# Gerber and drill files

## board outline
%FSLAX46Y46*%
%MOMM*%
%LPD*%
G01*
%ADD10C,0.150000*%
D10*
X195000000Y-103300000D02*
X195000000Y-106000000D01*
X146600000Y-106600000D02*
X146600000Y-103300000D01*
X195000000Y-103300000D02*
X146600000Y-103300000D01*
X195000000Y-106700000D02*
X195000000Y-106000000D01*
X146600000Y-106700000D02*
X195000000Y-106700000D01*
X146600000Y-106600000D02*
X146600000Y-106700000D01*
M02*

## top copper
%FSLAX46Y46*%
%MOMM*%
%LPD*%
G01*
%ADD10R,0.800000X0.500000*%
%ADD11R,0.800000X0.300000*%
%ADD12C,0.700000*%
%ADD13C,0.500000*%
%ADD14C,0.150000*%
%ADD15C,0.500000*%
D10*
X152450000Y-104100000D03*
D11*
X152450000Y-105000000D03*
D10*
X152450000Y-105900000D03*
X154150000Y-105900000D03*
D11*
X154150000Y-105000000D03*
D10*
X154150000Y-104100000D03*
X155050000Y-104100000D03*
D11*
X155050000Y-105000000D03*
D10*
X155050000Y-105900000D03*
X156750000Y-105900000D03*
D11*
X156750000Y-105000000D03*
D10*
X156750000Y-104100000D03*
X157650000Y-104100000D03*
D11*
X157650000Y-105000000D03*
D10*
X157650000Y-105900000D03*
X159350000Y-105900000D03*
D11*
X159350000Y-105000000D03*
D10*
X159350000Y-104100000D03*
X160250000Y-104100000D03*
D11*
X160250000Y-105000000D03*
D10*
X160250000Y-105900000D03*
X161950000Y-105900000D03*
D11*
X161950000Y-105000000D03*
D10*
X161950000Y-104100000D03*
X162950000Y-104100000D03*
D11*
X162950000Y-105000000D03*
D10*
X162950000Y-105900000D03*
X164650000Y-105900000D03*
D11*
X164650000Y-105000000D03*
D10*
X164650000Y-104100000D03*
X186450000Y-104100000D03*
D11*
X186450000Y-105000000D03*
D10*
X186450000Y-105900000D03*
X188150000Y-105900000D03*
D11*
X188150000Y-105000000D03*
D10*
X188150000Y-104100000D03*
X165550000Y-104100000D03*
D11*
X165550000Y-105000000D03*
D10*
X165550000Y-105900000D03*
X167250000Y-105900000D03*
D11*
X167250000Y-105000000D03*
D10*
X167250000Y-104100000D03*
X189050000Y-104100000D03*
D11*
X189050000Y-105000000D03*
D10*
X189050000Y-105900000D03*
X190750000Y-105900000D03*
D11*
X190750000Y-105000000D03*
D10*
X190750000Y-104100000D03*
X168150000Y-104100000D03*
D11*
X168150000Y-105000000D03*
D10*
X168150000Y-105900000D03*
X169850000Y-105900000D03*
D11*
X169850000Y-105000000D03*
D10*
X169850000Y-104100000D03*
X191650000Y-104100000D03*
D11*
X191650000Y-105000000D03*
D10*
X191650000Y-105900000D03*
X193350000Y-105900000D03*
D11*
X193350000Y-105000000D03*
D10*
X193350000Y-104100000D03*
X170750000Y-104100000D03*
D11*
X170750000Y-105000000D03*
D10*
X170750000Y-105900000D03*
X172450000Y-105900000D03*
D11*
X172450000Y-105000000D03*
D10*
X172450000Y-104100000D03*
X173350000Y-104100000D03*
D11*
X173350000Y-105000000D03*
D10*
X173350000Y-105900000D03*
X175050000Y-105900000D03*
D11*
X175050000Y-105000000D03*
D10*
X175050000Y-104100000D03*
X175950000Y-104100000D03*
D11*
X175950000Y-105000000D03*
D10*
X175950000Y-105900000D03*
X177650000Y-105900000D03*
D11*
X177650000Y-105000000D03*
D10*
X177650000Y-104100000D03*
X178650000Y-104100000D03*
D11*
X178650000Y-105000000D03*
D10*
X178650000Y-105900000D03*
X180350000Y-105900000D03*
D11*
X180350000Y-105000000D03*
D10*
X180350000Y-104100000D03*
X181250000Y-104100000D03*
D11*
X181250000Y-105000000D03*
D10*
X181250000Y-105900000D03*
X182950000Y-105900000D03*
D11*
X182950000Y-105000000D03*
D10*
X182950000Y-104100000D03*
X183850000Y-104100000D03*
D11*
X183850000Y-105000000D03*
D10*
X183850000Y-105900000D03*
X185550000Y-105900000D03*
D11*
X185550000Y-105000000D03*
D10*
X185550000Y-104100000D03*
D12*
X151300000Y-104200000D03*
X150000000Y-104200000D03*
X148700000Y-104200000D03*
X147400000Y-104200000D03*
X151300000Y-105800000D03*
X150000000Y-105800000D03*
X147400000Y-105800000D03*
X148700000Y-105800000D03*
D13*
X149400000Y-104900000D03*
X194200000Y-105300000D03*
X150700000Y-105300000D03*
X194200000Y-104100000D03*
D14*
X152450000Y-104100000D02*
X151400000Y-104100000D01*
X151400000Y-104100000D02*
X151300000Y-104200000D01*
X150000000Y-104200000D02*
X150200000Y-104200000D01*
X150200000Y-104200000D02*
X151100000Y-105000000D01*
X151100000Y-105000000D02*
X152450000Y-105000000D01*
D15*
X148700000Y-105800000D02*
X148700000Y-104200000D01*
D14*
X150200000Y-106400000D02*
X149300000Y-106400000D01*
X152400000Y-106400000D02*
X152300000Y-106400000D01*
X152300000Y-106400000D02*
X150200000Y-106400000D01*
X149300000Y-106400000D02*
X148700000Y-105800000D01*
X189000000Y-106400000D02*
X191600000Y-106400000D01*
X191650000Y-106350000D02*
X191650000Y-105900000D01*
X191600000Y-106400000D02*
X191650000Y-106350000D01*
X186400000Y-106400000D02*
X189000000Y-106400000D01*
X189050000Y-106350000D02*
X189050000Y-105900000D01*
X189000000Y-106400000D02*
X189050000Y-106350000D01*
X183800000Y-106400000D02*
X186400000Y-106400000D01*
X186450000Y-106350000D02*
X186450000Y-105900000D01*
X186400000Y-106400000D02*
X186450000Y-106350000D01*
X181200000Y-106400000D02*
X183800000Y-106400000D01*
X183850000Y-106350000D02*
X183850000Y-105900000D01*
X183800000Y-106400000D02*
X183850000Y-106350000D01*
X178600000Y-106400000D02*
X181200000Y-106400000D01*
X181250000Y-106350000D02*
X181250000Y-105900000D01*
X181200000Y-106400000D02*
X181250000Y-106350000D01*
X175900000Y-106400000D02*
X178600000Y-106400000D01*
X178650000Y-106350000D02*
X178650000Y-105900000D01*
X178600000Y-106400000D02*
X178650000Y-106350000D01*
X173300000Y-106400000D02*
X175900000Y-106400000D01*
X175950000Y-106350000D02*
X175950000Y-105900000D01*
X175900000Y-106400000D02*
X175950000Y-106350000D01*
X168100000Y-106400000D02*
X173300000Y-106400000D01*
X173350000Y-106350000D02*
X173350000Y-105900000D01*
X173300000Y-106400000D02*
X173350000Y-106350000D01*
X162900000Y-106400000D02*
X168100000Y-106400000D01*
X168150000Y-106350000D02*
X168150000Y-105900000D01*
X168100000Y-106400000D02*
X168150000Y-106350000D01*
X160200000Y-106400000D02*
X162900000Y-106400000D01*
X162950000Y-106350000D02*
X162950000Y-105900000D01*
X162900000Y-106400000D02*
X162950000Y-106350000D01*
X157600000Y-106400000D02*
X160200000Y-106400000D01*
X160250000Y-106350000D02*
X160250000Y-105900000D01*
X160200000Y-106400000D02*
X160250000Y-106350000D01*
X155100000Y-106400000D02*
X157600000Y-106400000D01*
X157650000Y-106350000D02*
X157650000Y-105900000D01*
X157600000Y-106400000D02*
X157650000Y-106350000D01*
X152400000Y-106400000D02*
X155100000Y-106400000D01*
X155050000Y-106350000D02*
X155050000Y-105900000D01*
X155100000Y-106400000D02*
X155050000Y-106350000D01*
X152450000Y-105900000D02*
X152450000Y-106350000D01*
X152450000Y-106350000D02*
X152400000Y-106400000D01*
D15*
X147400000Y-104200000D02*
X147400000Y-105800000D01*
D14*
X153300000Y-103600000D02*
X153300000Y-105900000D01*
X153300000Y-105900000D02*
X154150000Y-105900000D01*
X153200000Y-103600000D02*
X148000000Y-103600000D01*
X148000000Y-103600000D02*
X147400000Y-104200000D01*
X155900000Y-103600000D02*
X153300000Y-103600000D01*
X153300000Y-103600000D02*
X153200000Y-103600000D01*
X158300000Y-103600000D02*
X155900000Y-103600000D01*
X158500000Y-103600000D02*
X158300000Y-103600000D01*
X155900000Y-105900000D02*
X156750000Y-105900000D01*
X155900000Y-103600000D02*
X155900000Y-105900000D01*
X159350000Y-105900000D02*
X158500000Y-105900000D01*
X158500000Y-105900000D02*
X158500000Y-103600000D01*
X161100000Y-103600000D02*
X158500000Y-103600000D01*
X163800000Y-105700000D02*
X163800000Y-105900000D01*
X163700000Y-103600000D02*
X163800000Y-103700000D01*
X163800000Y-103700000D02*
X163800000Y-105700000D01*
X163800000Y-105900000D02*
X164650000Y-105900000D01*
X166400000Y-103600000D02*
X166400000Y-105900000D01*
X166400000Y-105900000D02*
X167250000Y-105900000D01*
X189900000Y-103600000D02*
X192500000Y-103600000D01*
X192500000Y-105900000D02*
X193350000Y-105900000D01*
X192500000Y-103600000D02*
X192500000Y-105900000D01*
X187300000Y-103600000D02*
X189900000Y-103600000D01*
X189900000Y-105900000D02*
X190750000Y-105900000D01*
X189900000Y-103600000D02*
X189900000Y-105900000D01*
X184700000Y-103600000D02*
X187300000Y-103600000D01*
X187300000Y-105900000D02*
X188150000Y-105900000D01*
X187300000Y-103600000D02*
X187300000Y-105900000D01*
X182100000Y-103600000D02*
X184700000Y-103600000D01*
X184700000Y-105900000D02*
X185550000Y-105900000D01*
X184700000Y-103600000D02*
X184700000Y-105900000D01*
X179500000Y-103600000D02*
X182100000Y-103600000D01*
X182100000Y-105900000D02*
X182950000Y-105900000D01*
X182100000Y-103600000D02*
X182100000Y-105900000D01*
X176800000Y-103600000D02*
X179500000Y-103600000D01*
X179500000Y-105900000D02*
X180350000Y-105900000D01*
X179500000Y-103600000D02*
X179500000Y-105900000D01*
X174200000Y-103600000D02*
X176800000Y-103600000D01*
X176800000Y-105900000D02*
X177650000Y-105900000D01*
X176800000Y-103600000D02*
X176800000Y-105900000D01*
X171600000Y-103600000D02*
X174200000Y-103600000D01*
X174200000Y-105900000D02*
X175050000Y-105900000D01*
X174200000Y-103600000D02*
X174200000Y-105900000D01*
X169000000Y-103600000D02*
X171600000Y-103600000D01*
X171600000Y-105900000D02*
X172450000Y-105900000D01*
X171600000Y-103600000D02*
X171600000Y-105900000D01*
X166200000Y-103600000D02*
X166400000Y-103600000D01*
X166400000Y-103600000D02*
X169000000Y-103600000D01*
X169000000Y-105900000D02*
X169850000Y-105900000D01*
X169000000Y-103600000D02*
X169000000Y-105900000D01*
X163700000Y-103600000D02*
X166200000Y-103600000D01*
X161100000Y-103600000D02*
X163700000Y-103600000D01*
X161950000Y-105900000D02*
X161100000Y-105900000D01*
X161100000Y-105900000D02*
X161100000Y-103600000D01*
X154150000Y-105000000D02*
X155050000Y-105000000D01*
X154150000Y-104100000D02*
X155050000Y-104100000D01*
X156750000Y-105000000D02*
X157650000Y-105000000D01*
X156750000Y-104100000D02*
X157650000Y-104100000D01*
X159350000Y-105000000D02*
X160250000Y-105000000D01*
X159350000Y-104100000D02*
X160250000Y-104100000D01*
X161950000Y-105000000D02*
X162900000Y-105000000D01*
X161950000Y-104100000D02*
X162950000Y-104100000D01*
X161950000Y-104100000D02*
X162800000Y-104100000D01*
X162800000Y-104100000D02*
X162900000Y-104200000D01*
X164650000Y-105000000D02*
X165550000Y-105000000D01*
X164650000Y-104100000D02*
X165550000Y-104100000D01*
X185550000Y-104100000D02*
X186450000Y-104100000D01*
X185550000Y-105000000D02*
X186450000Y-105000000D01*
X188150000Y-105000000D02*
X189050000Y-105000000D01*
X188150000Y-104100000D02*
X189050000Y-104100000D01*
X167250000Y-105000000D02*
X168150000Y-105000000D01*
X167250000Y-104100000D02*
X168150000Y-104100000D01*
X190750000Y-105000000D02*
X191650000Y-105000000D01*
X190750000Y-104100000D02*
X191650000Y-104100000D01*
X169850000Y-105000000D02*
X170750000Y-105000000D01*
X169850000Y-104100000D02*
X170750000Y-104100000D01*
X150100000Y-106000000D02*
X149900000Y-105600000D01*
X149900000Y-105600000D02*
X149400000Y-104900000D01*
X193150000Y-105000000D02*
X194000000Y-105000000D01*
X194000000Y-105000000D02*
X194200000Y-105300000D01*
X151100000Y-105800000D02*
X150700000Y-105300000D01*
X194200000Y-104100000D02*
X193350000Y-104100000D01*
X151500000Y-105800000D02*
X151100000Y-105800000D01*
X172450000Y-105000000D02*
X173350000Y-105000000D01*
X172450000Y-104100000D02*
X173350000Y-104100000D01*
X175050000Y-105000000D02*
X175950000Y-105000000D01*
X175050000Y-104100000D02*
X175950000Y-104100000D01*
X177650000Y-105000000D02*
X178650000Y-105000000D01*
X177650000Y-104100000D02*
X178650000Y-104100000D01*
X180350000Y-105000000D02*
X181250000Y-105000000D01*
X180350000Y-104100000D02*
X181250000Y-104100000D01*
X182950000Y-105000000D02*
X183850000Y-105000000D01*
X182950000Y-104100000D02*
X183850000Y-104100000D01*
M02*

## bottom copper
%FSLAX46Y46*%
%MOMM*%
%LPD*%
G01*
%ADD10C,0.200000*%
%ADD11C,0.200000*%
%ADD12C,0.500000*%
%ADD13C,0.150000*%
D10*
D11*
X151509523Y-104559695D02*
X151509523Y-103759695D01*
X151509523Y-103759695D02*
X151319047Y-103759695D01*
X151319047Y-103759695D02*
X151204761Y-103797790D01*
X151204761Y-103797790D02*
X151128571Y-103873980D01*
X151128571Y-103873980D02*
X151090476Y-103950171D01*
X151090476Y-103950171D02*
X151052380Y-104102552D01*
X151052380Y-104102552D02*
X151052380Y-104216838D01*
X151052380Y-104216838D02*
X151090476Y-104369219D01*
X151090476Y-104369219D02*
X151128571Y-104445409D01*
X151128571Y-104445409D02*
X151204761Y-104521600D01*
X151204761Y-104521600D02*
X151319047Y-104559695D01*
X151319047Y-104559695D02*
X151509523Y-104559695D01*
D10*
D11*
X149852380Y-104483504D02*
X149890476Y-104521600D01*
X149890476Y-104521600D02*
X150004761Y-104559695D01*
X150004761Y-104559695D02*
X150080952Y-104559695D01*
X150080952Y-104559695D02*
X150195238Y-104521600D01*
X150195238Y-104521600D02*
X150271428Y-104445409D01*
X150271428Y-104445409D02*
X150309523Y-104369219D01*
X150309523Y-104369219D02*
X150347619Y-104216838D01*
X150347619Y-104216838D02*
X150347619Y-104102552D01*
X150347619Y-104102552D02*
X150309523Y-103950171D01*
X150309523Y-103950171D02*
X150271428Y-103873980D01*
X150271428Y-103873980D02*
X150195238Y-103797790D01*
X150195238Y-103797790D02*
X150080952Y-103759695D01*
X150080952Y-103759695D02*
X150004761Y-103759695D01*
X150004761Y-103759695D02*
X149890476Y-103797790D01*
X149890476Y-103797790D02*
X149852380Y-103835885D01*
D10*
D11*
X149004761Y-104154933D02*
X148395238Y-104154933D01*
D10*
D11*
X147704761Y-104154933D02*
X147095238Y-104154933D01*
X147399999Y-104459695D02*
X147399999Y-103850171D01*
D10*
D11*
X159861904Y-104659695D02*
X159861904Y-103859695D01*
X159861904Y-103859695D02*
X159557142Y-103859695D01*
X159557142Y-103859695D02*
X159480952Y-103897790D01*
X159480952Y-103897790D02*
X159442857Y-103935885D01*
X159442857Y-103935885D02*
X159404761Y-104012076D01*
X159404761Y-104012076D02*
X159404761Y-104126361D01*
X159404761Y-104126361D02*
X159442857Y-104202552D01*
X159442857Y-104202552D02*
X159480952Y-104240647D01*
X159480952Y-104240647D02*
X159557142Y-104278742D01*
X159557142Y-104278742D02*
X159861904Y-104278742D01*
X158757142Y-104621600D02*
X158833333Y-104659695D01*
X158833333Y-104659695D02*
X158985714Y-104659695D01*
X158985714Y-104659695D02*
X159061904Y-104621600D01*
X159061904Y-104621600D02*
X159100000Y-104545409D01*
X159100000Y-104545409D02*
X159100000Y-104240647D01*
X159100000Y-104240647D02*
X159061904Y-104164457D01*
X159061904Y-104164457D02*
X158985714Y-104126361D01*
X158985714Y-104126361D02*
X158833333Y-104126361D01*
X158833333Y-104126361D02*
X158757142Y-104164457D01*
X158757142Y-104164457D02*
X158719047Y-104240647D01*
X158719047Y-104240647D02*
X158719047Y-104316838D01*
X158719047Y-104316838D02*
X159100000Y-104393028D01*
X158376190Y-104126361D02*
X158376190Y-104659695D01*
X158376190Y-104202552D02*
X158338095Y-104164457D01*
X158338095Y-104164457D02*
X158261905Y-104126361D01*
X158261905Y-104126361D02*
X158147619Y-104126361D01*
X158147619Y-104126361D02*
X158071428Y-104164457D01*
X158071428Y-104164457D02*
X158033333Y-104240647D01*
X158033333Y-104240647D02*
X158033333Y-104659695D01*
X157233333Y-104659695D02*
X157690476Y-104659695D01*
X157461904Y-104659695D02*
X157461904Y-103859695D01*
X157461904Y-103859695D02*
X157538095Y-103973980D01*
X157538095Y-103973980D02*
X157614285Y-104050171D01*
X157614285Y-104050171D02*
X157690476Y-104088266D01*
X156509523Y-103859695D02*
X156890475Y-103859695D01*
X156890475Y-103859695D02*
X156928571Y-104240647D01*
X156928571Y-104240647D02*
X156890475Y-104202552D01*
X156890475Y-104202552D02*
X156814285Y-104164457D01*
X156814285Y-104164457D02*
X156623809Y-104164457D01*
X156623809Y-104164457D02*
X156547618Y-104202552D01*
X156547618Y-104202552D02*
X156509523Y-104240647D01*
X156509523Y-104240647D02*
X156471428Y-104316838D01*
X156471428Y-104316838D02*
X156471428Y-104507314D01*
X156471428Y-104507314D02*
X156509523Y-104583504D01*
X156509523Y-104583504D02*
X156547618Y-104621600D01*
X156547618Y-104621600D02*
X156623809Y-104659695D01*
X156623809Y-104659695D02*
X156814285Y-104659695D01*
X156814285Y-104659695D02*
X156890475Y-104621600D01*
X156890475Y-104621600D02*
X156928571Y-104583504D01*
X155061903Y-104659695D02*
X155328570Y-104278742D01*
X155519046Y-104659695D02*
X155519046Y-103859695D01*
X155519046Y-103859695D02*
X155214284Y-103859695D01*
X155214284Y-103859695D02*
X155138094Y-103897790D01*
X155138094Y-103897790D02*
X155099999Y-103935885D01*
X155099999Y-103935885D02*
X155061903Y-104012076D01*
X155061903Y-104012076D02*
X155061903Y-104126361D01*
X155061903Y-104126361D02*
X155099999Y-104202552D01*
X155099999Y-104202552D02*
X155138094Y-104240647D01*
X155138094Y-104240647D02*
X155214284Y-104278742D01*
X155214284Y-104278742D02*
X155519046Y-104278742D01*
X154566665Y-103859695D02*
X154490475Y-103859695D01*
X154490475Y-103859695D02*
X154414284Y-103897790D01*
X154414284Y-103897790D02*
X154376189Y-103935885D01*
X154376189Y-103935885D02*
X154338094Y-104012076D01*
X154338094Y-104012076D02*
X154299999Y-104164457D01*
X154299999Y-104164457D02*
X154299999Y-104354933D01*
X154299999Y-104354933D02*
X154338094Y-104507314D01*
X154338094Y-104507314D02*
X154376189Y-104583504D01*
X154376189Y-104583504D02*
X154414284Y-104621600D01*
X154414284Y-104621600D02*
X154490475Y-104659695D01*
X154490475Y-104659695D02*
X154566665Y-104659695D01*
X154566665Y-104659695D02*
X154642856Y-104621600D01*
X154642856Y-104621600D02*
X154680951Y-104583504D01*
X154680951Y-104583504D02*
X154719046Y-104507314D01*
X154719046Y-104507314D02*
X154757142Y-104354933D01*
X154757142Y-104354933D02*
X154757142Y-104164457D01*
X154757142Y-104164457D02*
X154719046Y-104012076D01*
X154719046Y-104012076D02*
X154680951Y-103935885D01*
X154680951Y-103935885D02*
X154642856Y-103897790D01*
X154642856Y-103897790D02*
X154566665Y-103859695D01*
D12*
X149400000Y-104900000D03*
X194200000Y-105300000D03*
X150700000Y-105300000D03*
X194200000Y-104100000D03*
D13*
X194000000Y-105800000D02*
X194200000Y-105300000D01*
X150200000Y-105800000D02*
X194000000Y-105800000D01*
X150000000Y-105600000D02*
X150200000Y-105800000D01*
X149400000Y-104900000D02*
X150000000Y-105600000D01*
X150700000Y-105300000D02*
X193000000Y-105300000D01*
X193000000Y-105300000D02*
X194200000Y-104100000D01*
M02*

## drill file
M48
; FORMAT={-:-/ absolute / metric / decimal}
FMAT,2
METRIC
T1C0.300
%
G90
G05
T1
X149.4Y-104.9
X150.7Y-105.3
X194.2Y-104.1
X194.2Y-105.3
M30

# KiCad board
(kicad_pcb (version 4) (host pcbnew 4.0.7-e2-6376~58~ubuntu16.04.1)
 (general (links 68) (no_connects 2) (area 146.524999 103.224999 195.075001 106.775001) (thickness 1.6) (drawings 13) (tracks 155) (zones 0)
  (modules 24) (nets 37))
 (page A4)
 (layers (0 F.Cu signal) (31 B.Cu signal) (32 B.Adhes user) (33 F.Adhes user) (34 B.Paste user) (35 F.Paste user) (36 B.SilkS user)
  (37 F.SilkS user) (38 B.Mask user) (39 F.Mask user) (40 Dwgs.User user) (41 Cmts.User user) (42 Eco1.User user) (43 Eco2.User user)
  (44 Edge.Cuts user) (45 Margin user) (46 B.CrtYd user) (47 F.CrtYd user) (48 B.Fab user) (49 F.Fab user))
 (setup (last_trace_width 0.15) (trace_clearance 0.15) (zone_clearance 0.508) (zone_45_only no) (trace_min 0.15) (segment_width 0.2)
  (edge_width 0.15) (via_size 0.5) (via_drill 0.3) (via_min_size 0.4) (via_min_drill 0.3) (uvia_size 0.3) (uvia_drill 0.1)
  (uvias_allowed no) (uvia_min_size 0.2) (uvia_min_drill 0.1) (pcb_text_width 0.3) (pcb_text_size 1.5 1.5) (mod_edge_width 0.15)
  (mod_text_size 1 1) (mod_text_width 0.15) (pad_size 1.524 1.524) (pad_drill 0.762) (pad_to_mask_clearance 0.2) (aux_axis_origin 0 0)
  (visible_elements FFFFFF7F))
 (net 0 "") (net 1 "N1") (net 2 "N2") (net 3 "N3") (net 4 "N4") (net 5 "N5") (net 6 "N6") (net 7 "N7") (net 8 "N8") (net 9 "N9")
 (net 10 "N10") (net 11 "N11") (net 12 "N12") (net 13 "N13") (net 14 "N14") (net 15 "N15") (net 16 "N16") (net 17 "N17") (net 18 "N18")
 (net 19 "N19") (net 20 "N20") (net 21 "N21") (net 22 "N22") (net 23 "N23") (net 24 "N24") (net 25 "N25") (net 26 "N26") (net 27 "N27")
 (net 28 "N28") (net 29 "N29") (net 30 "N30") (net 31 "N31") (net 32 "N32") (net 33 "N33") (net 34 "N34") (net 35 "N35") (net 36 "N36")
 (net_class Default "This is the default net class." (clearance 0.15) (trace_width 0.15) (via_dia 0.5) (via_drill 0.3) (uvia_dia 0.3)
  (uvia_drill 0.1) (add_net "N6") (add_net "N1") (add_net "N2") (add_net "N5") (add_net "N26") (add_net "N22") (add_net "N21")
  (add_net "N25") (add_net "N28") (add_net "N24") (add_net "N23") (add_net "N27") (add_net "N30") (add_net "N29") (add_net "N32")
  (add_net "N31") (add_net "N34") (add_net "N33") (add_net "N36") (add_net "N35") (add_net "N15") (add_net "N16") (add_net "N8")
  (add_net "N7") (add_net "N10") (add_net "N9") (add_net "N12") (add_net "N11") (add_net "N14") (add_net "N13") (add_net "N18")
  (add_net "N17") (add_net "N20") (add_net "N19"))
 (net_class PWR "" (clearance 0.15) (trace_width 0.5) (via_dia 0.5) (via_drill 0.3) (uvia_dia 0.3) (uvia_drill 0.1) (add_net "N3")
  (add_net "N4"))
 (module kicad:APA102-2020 (layer F.Cu) (at 153.3 105)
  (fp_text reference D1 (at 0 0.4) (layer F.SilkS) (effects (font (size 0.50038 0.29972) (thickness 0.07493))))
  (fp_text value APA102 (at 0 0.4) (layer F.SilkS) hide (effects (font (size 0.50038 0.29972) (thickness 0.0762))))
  (pad 2 smd rect (at -0.85 -0.9) (size 0.8 0.5) (layers F.Cu F.Paste F.Mask) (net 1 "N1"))
  (pad 3 smd rect (at -0.85 0) (size 0.8 0.3) (layers F.Cu F.Paste F.Mask) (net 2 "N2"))
  (pad 4 smd rect (at -0.85 0.9) (size 0.8 0.5) (layers F.Cu F.Paste F.Mask) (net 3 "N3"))
  (pad 5 smd rect (at 0.85 0.9) (size 0.8 0.5) (layers F.Cu F.Paste F.Mask) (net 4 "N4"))
  (pad 6 smd rect (at 0.85 0) (size 0.8 0.3) (layers F.Cu F.Paste F.Mask) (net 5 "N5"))
  (pad 1 smd rect (at 0.85 -0.9) (size 0.8 0.5) (layers F.Cu F.Paste F.Mask) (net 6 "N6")))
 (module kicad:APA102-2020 (layer F.Cu) (at 155.9 105)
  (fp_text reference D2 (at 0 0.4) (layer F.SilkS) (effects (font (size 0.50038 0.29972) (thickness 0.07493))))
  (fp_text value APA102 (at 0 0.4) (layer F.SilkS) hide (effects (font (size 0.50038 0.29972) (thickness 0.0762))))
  (pad 2 smd rect (at -0.85 -0.9) (size 0.8 0.5) (layers F.Cu F.Paste F.Mask) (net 6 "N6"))
  (pad 3 smd rect (at -0.85 0) (size 0.8 0.3) (layers F.Cu F.Paste F.Mask) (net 5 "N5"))
  (pad 4 smd rect (at -0.85 0.9) (size 0.8 0.5) (layers F.Cu F.Paste F.Mask) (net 3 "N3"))
  (pad 5 smd rect (at 0.85 0.9) (size 0.8 0.5) (layers F.Cu F.Paste F.Mask) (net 4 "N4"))
  (pad 6 smd rect (at 0.85 0) (size 0.8 0.3) (layers F.Cu F.Paste F.Mask) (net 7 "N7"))
  (pad 1 smd rect (at 0.85 -0.9) (size 0.8 0.5) (layers F.Cu F.Paste F.Mask) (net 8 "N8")))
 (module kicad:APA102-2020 (layer F.Cu) (at 158.5 105)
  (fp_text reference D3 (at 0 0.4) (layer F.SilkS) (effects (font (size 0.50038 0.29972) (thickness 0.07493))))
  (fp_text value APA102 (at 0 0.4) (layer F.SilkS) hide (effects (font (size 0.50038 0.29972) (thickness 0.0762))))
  (pad 2 smd rect (at -0.85 -0.9) (size 0.8 0.5) (layers F.Cu F.Paste F.Mask) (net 8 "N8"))
  (pad 3 smd rect (at -0.85 0) (size 0.8 0.3) (layers F.Cu F.Paste F.Mask) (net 7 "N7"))
  (pad 4 smd rect (at -0.85 0.9) (size 0.8 0.5) (layers F.Cu F.Paste F.Mask) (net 3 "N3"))
  (pad 5 smd rect (at 0.85 0.9) (size 0.8 0.5) (layers F.Cu F.Paste F.Mask) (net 4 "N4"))
  (pad 6 smd rect (at 0.85 0) (size 0.8 0.3) (layers F.Cu F.Paste F.Mask) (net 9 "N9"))
  (pad 1 smd rect (at 0.85 -0.9) (size 0.8 0.5) (layers F.Cu F.Paste F.Mask) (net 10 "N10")))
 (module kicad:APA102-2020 (layer F.Cu) (at 161.1 105)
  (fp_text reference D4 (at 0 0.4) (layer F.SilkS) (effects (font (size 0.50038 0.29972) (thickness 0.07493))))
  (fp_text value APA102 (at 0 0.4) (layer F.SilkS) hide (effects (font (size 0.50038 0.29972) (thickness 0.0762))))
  (pad 2 smd rect (at -0.85 -0.9) (size 0.8 0.5) (layers F.Cu F.Paste F.Mask) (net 10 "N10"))
  (pad 3 smd rect (at -0.85 0) (size 0.8 0.3) (layers F.Cu F.Paste F.Mask) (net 9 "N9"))
  (pad 4 smd rect (at -0.85 0.9) (size 0.8 0.5) (layers F.Cu F.Paste F.Mask) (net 3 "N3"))
  (pad 5 smd rect (at 0.85 0.9) (size 0.8 0.5) (layers F.Cu F.Paste F.Mask) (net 4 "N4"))
  (pad 6 smd rect (at 0.85 0) (size 0.8 0.3) (layers F.Cu F.Paste F.Mask) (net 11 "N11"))
  (pad 1 smd rect (at 0.85 -0.9) (size 0.8 0.5) (layers F.Cu F.Paste F.Mask) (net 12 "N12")))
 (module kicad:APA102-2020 (layer F.Cu) (at 163.8 105)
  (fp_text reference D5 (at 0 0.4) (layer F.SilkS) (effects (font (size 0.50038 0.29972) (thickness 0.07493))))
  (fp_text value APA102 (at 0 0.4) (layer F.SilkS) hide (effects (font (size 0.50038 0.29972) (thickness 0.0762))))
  (pad 2 smd rect (at -0.85 -0.9) (size 0.8 0.5) (layers F.Cu F.Paste F.Mask) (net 12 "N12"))
  (pad 3 smd rect (at -0.85 0) (size 0.8 0.3) (layers F.Cu F.Paste F.Mask) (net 11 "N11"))
  (pad 4 smd rect (at -0.85 0.9) (size 0.8 0.5) (layers F.Cu F.Paste F.Mask) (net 3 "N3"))
  (pad 5 smd rect (at 0.85 0.9) (size 0.8 0.5) (layers F.Cu F.Paste F.Mask) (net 4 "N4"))
  (pad 6 smd rect (at 0.85 0) (size 0.8 0.3) (layers F.Cu F.Paste F.Mask) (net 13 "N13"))
  (pad 1 smd rect (at 0.85 -0.9) (size 0.8 0.5) (layers F.Cu F.Paste F.Mask) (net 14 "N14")))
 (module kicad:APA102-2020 (layer F.Cu) (at 187.3 105)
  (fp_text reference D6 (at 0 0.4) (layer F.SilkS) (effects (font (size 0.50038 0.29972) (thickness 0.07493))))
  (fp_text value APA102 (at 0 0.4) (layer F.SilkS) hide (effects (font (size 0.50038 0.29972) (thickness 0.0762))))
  (pad 2 smd rect (at -0.85 -0.9) (size 0.8 0.5) (layers F.Cu F.Paste F.Mask) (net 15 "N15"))
  (pad 3 smd rect (at -0.85 0) (size 0.8 0.3) (layers F.Cu F.Paste F.Mask) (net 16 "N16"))
  (pad 4 smd rect (at -0.85 0.9) (size 0.8 0.5) (layers F.Cu F.Paste F.Mask) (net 3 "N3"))
  (pad 5 smd rect (at 0.85 0.9) (size 0.8 0.5) (layers F.Cu F.Paste F.Mask) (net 4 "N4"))
  (pad 6 smd rect (at 0.85 0) (size 0.8 0.3) (layers F.Cu F.Paste F.Mask) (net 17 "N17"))
  (pad 1 smd rect (at 0.85 -0.9) (size 0.8 0.5) (layers F.Cu F.Paste F.Mask) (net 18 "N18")))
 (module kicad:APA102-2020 (layer F.Cu) (at 166.4 105)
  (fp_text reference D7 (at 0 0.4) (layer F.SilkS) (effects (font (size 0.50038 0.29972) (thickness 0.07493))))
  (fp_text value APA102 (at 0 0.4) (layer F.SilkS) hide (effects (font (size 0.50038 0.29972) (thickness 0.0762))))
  (pad 2 smd rect (at -0.85 -0.9) (size 0.8 0.5) (layers F.Cu F.Paste F.Mask) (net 14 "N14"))
  (pad 3 smd rect (at -0.85 0) (size 0.8 0.3) (layers F.Cu F.Paste F.Mask) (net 13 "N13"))
  (pad 4 smd rect (at -0.85 0.9) (size 0.8 0.5) (layers F.Cu F.Paste F.Mask) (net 3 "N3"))
  (pad 5 smd rect (at 0.85 0.9) (size 0.8 0.5) (layers F.Cu F.Paste F.Mask) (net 4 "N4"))
  (pad 6 smd rect (at 0.85 0) (size 0.8 0.3) (layers F.Cu F.Paste F.Mask) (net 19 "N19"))
  (pad 1 smd rect (at 0.85 -0.9) (size 0.8 0.5) (layers F.Cu F.Paste F.Mask) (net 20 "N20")))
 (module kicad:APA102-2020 (layer F.Cu) (at 189.9 105)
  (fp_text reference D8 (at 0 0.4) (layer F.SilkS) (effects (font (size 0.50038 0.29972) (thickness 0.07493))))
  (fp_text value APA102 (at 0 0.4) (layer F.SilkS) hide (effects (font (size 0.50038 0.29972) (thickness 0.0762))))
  (pad 2 smd rect (at -0.85 -0.9) (size 0.8 0.5) (layers F.Cu F.Paste F.Mask) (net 18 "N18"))
  (pad 3 smd rect (at -0.85 0) (size 0.8 0.3) (layers F.Cu F.Paste F.Mask) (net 17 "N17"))
  (pad 4 smd rect (at -0.85 0.9) (size 0.8 0.5) (layers F.Cu F.Paste F.Mask) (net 3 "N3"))
  (pad 5 smd rect (at 0.85 0.9) (size 0.8 0.5) (layers F.Cu F.Paste F.Mask) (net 4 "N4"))
  (pad 6 smd rect (at 0.85 0) (size 0.8 0.3) (layers F.Cu F.Paste F.Mask) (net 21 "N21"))
  (pad 1 smd rect (at 0.85 -0.9) (size 0.8 0.5) (layers F.Cu F.Paste F.Mask) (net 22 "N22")))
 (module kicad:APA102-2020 (layer F.Cu) (at 169 105)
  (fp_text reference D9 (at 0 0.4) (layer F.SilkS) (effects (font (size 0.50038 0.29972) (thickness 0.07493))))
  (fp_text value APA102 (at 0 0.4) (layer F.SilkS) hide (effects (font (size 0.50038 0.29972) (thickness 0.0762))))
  (pad 2 smd rect (at -0.85 -0.9) (size 0.8 0.5) (layers F.Cu F.Paste F.Mask) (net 20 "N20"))
  (pad 3 smd rect (at -0.85 0) (size 0.8 0.3) (layers F.Cu F.Paste F.Mask) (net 19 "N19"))
  (pad 4 smd rect (at -0.85 0.9) (size 0.8 0.5) (layers F.Cu F.Paste F.Mask) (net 3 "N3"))
  (pad 5 smd rect (at 0.85 0.9) (size 0.8 0.5) (layers F.Cu F.Paste F.Mask) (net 4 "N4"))
  (pad 6 smd rect (at 0.85 0) (size 0.8 0.3) (layers F.Cu F.Paste F.Mask) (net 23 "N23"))
  (pad 1 smd rect (at 0.85 -0.9) (size 0.8 0.5) (layers F.Cu F.Paste F.Mask) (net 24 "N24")))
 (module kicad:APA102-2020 (layer F.Cu) (at 192.5 105)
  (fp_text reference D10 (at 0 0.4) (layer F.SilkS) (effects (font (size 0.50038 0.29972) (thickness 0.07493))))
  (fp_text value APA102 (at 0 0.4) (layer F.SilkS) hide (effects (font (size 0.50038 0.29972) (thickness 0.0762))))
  (pad 2 smd rect (at -0.85 -0.9) (size 0.8 0.5) (layers F.Cu F.Paste F.Mask) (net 22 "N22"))
  (pad 3 smd rect (at -0.85 0) (size 0.8 0.3) (layers F.Cu F.Paste F.Mask) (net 21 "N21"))
  (pad 4 smd rect (at -0.85 0.9) (size 0.8 0.5) (layers F.Cu F.Paste F.Mask) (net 3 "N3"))
  (pad 5 smd rect (at 0.85 0.9) (size 0.8 0.5) (layers F.Cu F.Paste F.Mask) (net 4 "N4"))
  (pad 6 smd rect (at 0.85 0) (size 0.8 0.3) (layers F.Cu F.Paste F.Mask) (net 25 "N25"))
  (pad 1 smd rect (at 0.85 -0.9) (size 0.8 0.5) (layers F.Cu F.Paste F.Mask) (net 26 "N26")))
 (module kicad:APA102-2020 (layer F.Cu) (at 171.6 105)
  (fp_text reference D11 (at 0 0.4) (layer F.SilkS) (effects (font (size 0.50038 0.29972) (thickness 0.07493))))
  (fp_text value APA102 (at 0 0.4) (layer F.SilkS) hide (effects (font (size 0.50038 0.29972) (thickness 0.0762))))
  (pad 2 smd rect (at -0.85 -0.9) (size 0.8 0.5) (layers F.Cu F.Paste F.Mask) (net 24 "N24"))
  (pad 3 smd rect (at -0.85 0) (size 0.8 0.3) (layers F.Cu F.Paste F.Mask) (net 23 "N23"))
  (pad 4 smd rect (at -0.85 0.9) (size 0.8 0.5) (layers F.Cu F.Paste F.Mask) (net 3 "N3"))
  (pad 5 smd rect (at 0.85 0.9) (size 0.8 0.5) (layers F.Cu F.Paste F.Mask) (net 4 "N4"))
  (pad 6 smd rect (at 0.85 0) (size 0.8 0.3) (layers F.Cu F.Paste F.Mask) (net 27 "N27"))
  (pad 1 smd rect (at 0.85 -0.9) (size 0.8 0.5) (layers F.Cu F.Paste F.Mask) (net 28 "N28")))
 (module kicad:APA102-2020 (layer F.Cu) (at 174.2 105)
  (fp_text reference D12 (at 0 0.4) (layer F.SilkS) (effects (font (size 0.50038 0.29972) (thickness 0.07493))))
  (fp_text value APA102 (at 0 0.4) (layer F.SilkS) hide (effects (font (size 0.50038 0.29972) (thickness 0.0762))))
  (pad 2 smd rect (at -0.85 -0.9) (size 0.8 0.5) (layers F.Cu F.Paste F.Mask) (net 28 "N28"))
  (pad 3 smd rect (at -0.85 0) (size 0.8 0.3) (layers F.Cu F.Paste F.Mask) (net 27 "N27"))
  (pad 4 smd rect (at -0.85 0.9) (size 0.8 0.5) (layers F.Cu F.Paste F.Mask) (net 3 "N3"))
  (pad 5 smd rect (at 0.85 0.9) (size 0.8 0.5) (layers F.Cu F.Paste F.Mask) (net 4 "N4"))
  (pad 6 smd rect (at 0.85 0) (size 0.8 0.3) (layers F.Cu F.Paste F.Mask) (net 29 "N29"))
  (pad 1 smd rect (at 0.85 -0.9) (size 0.8 0.5) (layers F.Cu F.Paste F.Mask) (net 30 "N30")))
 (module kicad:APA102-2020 (layer F.Cu) (at 176.8 105)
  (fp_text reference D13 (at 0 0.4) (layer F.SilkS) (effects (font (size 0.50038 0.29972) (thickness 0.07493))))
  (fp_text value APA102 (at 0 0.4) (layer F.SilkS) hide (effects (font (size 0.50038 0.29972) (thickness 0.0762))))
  (pad 2 smd rect (at -0.85 -0.9) (size 0.8 0.5) (layers F.Cu F.Paste F.Mask) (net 30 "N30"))
  (pad 3 smd rect (at -0.85 0) (size 0.8 0.3) (layers F.Cu F.Paste F.Mask) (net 29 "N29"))
  (pad 4 smd rect (at -0.85 0.9) (size 0.8 0.5) (layers F.Cu F.Paste F.Mask) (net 3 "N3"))
  (pad 5 smd rect (at 0.85 0.9) (size 0.8 0.5) (layers F.Cu F.Paste F.Mask) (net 4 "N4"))
  (pad 6 smd rect (at 0.85 0) (size 0.8 0.3) (layers F.Cu F.Paste F.Mask) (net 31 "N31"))
  (pad 1 smd rect (at 0.85 -0.9) (size 0.8 0.5) (layers F.Cu F.Paste F.Mask) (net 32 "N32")))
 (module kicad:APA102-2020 (layer F.Cu) (at 179.5 105)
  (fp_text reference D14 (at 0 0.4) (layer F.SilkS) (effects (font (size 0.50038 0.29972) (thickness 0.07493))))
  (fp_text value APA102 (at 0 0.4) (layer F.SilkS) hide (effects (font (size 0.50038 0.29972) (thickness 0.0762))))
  (pad 2 smd rect (at -0.85 -0.9) (size 0.8 0.5) (layers F.Cu F.Paste F.Mask) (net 32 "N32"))
  (pad 3 smd rect (at -0.85 0) (size 0.8 0.3) (layers F.Cu F.Paste F.Mask) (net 31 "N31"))
  (pad 4 smd rect (at -0.85 0.9) (size 0.8 0.5) (layers F.Cu F.Paste F.Mask) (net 3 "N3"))
  (pad 5 smd rect (at 0.85 0.9) (size 0.8 0.5) (layers F.Cu F.Paste F.Mask) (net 4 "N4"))
  (pad 6 smd rect (at 0.85 0) (size 0.8 0.3) (layers F.Cu F.Paste F.Mask) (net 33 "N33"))
  (pad 1 smd rect (at 0.85 -0.9) (size 0.8 0.5) (layers F.Cu F.Paste F.Mask) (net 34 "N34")))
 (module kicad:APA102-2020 (layer F.Cu) (at 182.1 105)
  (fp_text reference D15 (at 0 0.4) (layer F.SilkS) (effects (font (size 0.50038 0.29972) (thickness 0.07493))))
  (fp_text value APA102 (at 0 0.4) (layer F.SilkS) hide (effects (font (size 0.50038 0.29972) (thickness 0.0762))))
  (pad 2 smd rect (at -0.85 -0.9) (size 0.8 0.5) (layers F.Cu F.Paste F.Mask) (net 34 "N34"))
  (pad 3 smd rect (at -0.85 0) (size 0.8 0.3) (layers F.Cu F.Paste F.Mask) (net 33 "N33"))
  (pad 4 smd rect (at -0.85 0.9) (size 0.8 0.5) (layers F.Cu F.Paste F.Mask) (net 3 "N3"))
  (pad 5 smd rect (at 0.85 0.9) (size 0.8 0.5) (layers F.Cu F.Paste F.Mask) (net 4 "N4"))
  (pad 6 smd rect (at 0.85 0) (size 0.8 0.3) (layers F.Cu F.Paste F.Mask) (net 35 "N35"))
  (pad 1 smd rect (at 0.85 -0.9) (size 0.8 0.5) (layers F.Cu F.Paste F.Mask) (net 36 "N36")))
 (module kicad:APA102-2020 (layer F.Cu) (at 184.7 105)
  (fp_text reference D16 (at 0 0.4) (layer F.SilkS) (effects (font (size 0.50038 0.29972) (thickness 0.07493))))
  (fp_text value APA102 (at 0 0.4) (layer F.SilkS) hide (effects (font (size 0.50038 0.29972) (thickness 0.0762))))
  (pad 2 smd rect (at -0.85 -0.9) (size 0.8 0.5) (layers F.Cu F.Paste F.Mask) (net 36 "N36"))
  (pad 3 smd rect (at -0.85 0) (size 0.8 0.3) (layers F.Cu F.Paste F.Mask) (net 35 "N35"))
  (pad 4 smd rect (at -0.85 0.9) (size 0.8 0.5) (layers F.Cu F.Paste F.Mask) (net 3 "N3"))
  (pad 5 smd rect (at 0.85 0.9) (size 0.8 0.5) (layers F.Cu F.Paste F.Mask) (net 4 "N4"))
  (pad 6 smd rect (at 0.85 0) (size 0.8 0.3) (layers F.Cu F.Paste F.Mask) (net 16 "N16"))
  (pad 1 smd rect (at 0.85 -0.9) (size 0.8 0.5) (layers F.Cu F.Paste F.Mask) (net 15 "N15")))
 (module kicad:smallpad (layer F.Cu) (at 151.3 104.2)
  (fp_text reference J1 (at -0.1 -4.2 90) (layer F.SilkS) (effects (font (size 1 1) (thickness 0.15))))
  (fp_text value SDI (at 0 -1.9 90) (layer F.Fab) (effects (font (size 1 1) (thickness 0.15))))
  (pad 1 smd circle (at 0 0) (size 0.7 0.7) (layers F.Cu F.Paste F.Mask) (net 1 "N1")))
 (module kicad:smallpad (layer F.Cu) (at 150 104.2)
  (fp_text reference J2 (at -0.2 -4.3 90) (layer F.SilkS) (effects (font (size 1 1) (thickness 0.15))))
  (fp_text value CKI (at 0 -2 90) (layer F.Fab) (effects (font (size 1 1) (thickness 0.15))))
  (pad 1 smd circle (at 0 0) (size 0.7 0.7) (layers F.Cu F.Paste F.Mask) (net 2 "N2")))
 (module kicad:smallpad (layer F.Cu) (at 148.7 104.2)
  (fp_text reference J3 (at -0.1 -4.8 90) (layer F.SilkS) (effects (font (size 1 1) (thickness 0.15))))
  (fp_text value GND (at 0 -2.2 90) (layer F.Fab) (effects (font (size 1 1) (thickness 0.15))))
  (pad 1 smd circle (at 0 0) (size 0.7 0.7) (layers F.Cu F.Paste F.Mask) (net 3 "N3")))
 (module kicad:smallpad (layer F.Cu) (at 147.4 104.2)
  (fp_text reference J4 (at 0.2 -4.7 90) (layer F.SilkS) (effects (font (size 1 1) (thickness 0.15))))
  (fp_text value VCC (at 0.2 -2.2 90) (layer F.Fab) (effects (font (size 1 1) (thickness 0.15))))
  (pad 1 smd circle (at 0 0) (size 0.7 0.7) (layers F.Cu F.Paste F.Mask) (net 4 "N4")))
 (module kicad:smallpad (layer F.Cu) (at 151.3 105.8)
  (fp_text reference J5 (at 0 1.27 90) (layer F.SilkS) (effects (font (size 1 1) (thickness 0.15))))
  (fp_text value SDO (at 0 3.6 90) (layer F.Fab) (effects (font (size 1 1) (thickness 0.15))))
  (pad 1 smd circle (at 0 0) (size 0.7 0.7) (layers F.Cu F.Paste F.Mask) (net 26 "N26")))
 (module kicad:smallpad (layer F.Cu) (at 150 105.8)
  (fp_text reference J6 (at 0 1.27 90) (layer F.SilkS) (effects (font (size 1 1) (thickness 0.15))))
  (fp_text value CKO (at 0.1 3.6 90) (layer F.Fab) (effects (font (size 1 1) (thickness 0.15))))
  (pad 1 smd circle (at 0 0) (size 0.7 0.7) (layers F.Cu F.Paste F.Mask) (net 25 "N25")))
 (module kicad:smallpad (layer F.Cu) (at 147.4 105.8)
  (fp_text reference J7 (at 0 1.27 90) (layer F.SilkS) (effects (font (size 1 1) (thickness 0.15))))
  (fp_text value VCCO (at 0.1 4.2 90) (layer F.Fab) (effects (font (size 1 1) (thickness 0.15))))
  (pad 1 smd circle (at 0 0) (size 0.7 0.7) (layers F.Cu F.Paste F.Mask) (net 4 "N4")))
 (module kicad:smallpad (layer F.Cu) (at 148.7 105.8)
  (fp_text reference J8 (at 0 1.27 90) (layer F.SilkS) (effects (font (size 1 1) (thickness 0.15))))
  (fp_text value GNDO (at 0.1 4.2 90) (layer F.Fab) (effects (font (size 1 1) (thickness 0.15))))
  (pad 1 smd circle (at 0 0) (size 0.7 0.7) (layers F.Cu F.Paste F.Mask) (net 3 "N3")))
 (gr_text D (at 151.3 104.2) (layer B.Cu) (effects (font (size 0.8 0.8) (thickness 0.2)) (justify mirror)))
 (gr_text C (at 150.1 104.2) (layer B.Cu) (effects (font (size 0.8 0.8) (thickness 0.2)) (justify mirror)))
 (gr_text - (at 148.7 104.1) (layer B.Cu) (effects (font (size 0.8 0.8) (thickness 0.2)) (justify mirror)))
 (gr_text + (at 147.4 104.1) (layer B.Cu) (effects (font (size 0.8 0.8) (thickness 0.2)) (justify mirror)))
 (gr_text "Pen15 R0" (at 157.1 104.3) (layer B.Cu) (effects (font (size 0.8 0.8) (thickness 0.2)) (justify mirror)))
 (gr_line (start 195 103.3) (end 195 106) (angle 90) (layer Edge.Cuts) (width 0.15))
 (gr_line (start 146.6 106.6) (end 146.6 103.3) (angle 90) (layer Edge.Cuts) (width 0.15))
 (gr_line (start 195 103.3) (end 146.6 103.3) (angle 90) (layer Edge.Cuts) (width 0.15))
 (gr_line (start 195 106.7) (end 195 106) (angle 90) (layer Edge.Cuts) (width 0.15))
 (gr_line (start 146.6 106.7) (end 195 106.7) (angle 90) (layer Edge.Cuts) (width 0.15))
 (gr_line (start 146.6 106.6) (end 146.6 106.7) (angle 90) (layer Edge.Cuts) (width 0.15))
 (segment (start 152.45 104.1) (end 151.4 104.1) (width 0.15) (layer F.Cu) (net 1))
 (segment (start 151.4 104.1) (end 151.3 104.2) (width 0.15) (layer F.Cu) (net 1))
 (segment (start 150 104.2) (end 150.2 104.2) (width 0.15) (layer F.Cu) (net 2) (status 30))
 (segment (start 150.2 104.2) (end 151.1 105) (width 0.15) (layer F.Cu) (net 2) (status 10))
 (segment (start 151.1 105) (end 152.45 105) (width 0.15) (layer F.Cu) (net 2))
 (segment (start 148.7 105.8) (end 148.7 104.2) (width 0.5) (layer F.Cu) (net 3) (status 10))
 (segment (start 150.2 106.4) (end 149.3 106.4) (width 0.15) (layer F.Cu) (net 3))
 (segment (start 152.4 106.4) (end 152.3 106.4) (width 0.15) (layer F.Cu) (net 3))
 (segment (start 152.3 106.4) (end 150.2 106.4) (width 0.15) (layer F.Cu) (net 3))
 (segment (start 149.3 106.4) (end 148.7 105.8) (width 0.15) (layer F.Cu) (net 3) (status 20))
 (segment (start 189 106.4) (end 191.6 106.4) (width 0.15) (layer F.Cu) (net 3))
 (segment (start 191.65 106.35) (end 191.65 105.9) (width 0.15) (layer F.Cu) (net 3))
 (segment (start 191.6 106.4) (end 191.65 106.35) (width 0.15) (layer F.Cu) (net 3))
 (segment (start 186.4 106.4) (end 189 106.4) (width 0.15) (layer F.Cu) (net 3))
 (segment (start 189.05 106.35) (end 189.05 105.9) (width 0.15) (layer F.Cu) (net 3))
 (segment (start 189 106.4) (end 189.05 106.35) (width 0.15) (layer F.Cu) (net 3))
 (segment (start 183.8 106.4) (end 186.4 106.4) (width 0.15) (layer F.Cu) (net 3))
 (segment (start 186.45 106.35) (end 186.45 105.9) (width 0.15) (layer F.Cu) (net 3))
 (segment (start 186.4 106.4) (end 186.45 106.35) (width 0.15) (layer F.Cu) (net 3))
 (segment (start 181.2 106.4) (end 183.8 106.4) (width 0.15) (layer F.Cu) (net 3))
 (segment (start 183.85 106.35) (end 183.85 105.9) (width 0.15) (layer F.Cu) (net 3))
 (segment (start 183.8 106.4) (end 183.85 106.35) (width 0.15) (layer F.Cu) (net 3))
 (segment (start 178.6 106.4) (end 181.2 106.4) (width 0.15) (layer F.Cu) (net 3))
 (segment (start 181.25 106.35) (end 181.25 105.9) (width 0.15) (layer F.Cu) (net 3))
 (segment (start 181.2 106.4) (end 181.25 106.35) (width 0.15) (layer F.Cu) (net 3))
 (segment (start 175.9 106.4) (end 178.6 106.4) (width 0.15) (layer F.Cu) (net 3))
 (segment (start 178.65 106.35) (end 178.65 105.9) (width 0.15) (layer F.Cu) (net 3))
 (segment (start 178.6 106.4) (end 178.65 106.35) (width 0.15) (layer F.Cu) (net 3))
 (segment (start 173.3 106.4) (end 175.9 106.4) (width 0.15) (layer F.Cu) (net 3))
 (segment (start 175.95 106.35) (end 175.95 105.9) (width 0.15) (layer F.Cu) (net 3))
 (segment (start 175.9 106.4) (end 175.95 106.35) (width 0.15) (layer F.Cu) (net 3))
 (segment (start 168.1 106.4) (end 173.3 106.4) (width 0.15) (layer F.Cu) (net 3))
 (segment (start 173.35 106.35) (end 173.35 105.9) (width 0.15) (layer F.Cu) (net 3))
 (segment (start 173.3 106.4) (end 173.35 106.35) (width 0.15) (layer F.Cu) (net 3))
 (segment (start 162.9 106.4) (end 168.1 106.4) (width 0.15) (layer F.Cu) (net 3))
 (segment (start 168.15 106.35) (end 168.15 105.9) (width 0.15) (layer F.Cu) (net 3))
 (segment (start 168.1 106.4) (end 168.15 106.35) (width 0.15) (layer F.Cu) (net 3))
 (segment (start 160.2 106.4) (end 162.9 106.4) (width 0.15) (layer F.Cu) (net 3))
 (segment (start 162.95 106.35) (end 162.95 105.9) (width 0.15) (layer F.Cu) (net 3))
 (segment (start 162.9 106.4) (end 162.95 106.35) (width 0.15) (layer F.Cu) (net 3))
 (segment (start 157.6 106.4) (end 160.2 106.4) (width 0.15) (layer F.Cu) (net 3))
 (segment (start 160.25 106.35) (end 160.25 105.9) (width 0.15) (layer F.Cu) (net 3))
 (segment (start 160.2 106.4) (end 160.25 106.35) (width 0.15) (layer F.Cu) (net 3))
 (segment (start 155.1 106.4) (end 157.6 106.4) (width 0.15) (layer F.Cu) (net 3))
 (segment (start 157.65 106.35) (end 157.65 105.9) (width 0.15) (layer F.Cu) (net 3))
 (segment (start 157.6 106.4) (end 157.65 106.35) (width 0.15) (layer F.Cu) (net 3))
 (segment (start 152.4 106.4) (end 155.1 106.4) (width 0.15) (layer F.Cu) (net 3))
 (segment (start 155.05 106.35) (end 155.05 105.9) (width 0.15) (layer F.Cu) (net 3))
 (segment (start 155.1 106.4) (end 155.05 106.35) (width 0.15) (layer F.Cu) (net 3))
 (segment (start 152.45 105.9) (end 152.45 106.35) (width 0.15) (layer F.Cu) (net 3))
 (segment (start 152.45 106.35) (end 152.4 106.4) (width 0.15) (layer F.Cu) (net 3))
 (segment (start 147.4 104.2) (end 147.4 105.8) (width 0.5) (layer F.Cu) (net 4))
 (segment (start 153.3 103.6) (end 153.3 105.9) (width 0.15) (layer F.Cu) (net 4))
 (segment (start 153.3 105.9) (end 154.15 105.9) (width 0.15) (layer F.Cu) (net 4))
 (segment (start 153.2 103.6) (end 148 103.6) (width 0.15) (layer F.Cu) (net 4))
 (segment (start 148 103.6) (end 147.4 104.2) (width 0.15) (layer F.Cu) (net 4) (status 20))
 (segment (start 155.9 103.6) (end 153.3 103.6) (width 0.15) (layer F.Cu) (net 4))
 (segment (start 153.3 103.6) (end 153.2 103.6) (width 0.15) (layer F.Cu) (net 4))
 (segment (start 158.3 103.6) (end 155.9 103.6) (width 0.15) (layer F.Cu) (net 4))
 (segment (start 158.5 103.6) (end 158.3 103.6) (width 0.15) (layer F.Cu) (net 4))
 (segment (start 155.9 105.9) (end 156.75 105.9) (width 0.15) (layer F.Cu) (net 4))
 (segment (start 155.9 103.6) (end 155.9 105.9) (width 0.15) (layer F.Cu) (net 4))
 (segment (start 159.35 105.9) (end 158.5 105.9) (width 0.15) (layer F.Cu) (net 4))
 (segment (start 158.5 105.9) (end 158.5 103.6) (width 0.15) (layer F.Cu) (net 4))
 (segment (start 161.1 103.6) (end 158.5 103.6) (width 0.15) (layer F.Cu) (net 4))
 (segment (start 163.8 105.7) (end 163.8 105.9) (width 0.15) (layer F.Cu) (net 4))
 (segment (start 163.7 103.6) (end 163.8 103.7) (width 0.15) (layer F.Cu) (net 4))
 (segment (start 163.8 103.7) (end 163.8 105.7) (width 0.15) (layer F.Cu) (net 4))
 (segment (start 163.8 105.9) (end 164.65 105.9) (width 0.15) (layer F.Cu) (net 4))
 (segment (start 166.4 103.6) (end 166.4 105.9) (width 0.15) (layer F.Cu) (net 4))
 (segment (start 166.4 105.9) (end 167.25 105.9) (width 0.15) (layer F.Cu) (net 4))
 (segment (start 189.9 103.6) (end 192.5 103.6) (width 0.15) (layer F.Cu) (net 4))
 (segment (start 192.5 105.9) (end 193.35 105.9) (width 0.15) (layer F.Cu) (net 4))
 (segment (start 192.5 103.6) (end 192.5 105.9) (width 0.15) (layer F.Cu) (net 4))
 (segment (start 187.3 103.6) (end 189.9 103.6) (width 0.15) (layer F.Cu) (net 4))
 (segment (start 189.9 105.9) (end 190.75 105.9) (width 0.15) (layer F.Cu) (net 4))
 (segment (start 189.9 103.6) (end 189.9 105.9) (width 0.15) (layer F.Cu) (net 4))
 (segment (start 184.7 103.6) (end 187.3 103.6) (width 0.15) (layer F.Cu) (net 4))
 (segment (start 187.3 105.9) (end 188.15 105.9) (width 0.15) (layer F.Cu) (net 4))
 (segment (start 187.3 103.6) (end 187.3 105.9) (width 0.15) (layer F.Cu) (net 4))
 (segment (start 182.1 103.6) (end 184.7 103.6) (width 0.15) (layer F.Cu) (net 4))
 (segment (start 184.7 105.9) (end 185.55 105.9) (width 0.15) (layer F.Cu) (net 4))
 (segment (start 184.7 103.6) (end 184.7 105.9) (width 0.15) (layer F.Cu) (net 4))
 (segment (start 179.5 103.6) (end 182.1 103.6) (width 0.15) (layer F.Cu) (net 4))
 (segment (start 182.1 105.9) (end 182.95 105.9) (width 0.15) (layer F.Cu) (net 4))
 (segment (start 182.1 103.6) (end 182.1 105.9) (width 0.15) (layer F.Cu) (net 4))
 (segment (start 176.8 103.6) (end 179.5 103.6) (width 0.15) (layer F.Cu) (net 4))
 (segment (start 179.5 105.9) (end 180.35 105.9) (width 0.15) (layer F.Cu) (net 4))
 (segment (start 179.5 103.6) (end 179.5 105.9) (width 0.15) (layer F.Cu) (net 4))
 (segment (start 174.2 103.6) (end 176.8 103.6) (width 0.15) (layer F.Cu) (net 4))
 (segment (start 176.8 105.9) (end 177.65 105.9) (width 0.15) (layer F.Cu) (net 4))
 (segment (start 176.8 103.6) (end 176.8 105.9) (width 0.15) (layer F.Cu) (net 4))
 (segment (start 171.6 103.6) (end 174.2 103.6) (width 0.15) (layer F.Cu) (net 4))
 (segment (start 174.2 105.9) (end 175.05 105.9) (width 0.15) (layer F.Cu) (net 4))
 (segment (start 174.2 103.6) (end 174.2 105.9) (width 0.15) (layer F.Cu) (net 4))
 (segment (start 169 103.6) (end 171.6 103.6) (width 0.15) (layer F.Cu) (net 4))
 (segment (start 171.6 105.9) (end 172.45 105.9) (width 0.15) (layer F.Cu) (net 4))
 (segment (start 171.6 103.6) (end 171.6 105.9) (width 0.15) (layer F.Cu) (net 4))
 (segment (start 166.2 103.6) (end 166.4 103.6) (width 0.15) (layer F.Cu) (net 4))
 (segment (start 166.4 103.6) (end 169 103.6) (width 0.15) (layer F.Cu) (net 4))
 (segment (start 169 105.9) (end 169.85 105.9) (width 0.15) (layer F.Cu) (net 4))
 (segment (start 169 103.6) (end 169 105.9) (width 0.15) (layer F.Cu) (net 4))
 (segment (start 163.7 103.6) (end 166.2 103.6) (width 0.15) (layer F.Cu) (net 4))
 (segment (start 161.1 103.6) (end 163.7 103.6) (width 0.15) (layer F.Cu) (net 4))
 (segment (start 161.95 105.9) (end 161.1 105.9) (width 0.15) (layer F.Cu) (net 4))
 (segment (start 161.1 105.9) (end 161.1 103.6) (width 0.15) (layer F.Cu) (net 4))
 (segment (start 154.15 105) (end 155.05 105) (width 0.15) (layer F.Cu) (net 5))
 (segment (start 154.15 104.1) (end 155.05 104.1) (width 0.15) (layer F.Cu) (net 6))
 (segment (start 156.75 105) (end 157.65 105) (width 0.15) (layer F.Cu) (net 7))
 (segment (start 156.75 104.1) (end 157.65 104.1) (width 0.15) (layer F.Cu) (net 8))
 (segment (start 159.35 105) (end 160.25 105) (width 0.15) (layer F.Cu) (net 9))
 (segment (start 159.35 104.1) (end 160.25 104.1) (width 0.15) (layer F.Cu) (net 10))
 (segment (start 161.95 105) (end 162.9 105) (width 0.15) (layer F.Cu) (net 11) (status 20))
 (segment (start 161.95 104.1) (end 162.95 104.1) (width 0.15) (layer F.Cu) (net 12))
 (segment (start 161.95 104.1) (end 162.8 104.1) (width 0.15) (layer F.Cu) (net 12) (status 20))
 (segment (start 162.8 104.1) (end 162.9 104.2) (width 0.15) (layer F.Cu) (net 12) (status 30))
 (segment (start 164.65 105) (end 165.55 105) (width 0.15) (layer F.Cu) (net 13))
 (segment (start 164.65 104.1) (end 165.55 104.1) (width 0.15) (layer F.Cu) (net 14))
 (segment (start 185.55 104.1) (end 186.45 104.1) (width 0.15) (layer F.Cu) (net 15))
 (segment (start 185.55 105) (end 186.45 105) (width 0.15) (layer F.Cu) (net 16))
 (segment (start 188.15 105) (end 189.05 105) (width 0.15) (layer F.Cu) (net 17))
 (segment (start 188.15 104.1) (end 189.05 104.1) (width 0.15) (layer F.Cu) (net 18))
 (segment (start 167.25 105) (end 168.15 105) (width 0.15) (layer F.Cu) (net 19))
 (segment (start 167.25 104.1) (end 168.15 104.1) (width 0.15) (layer F.Cu) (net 20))
 (segment (start 190.75 105) (end 191.65 105) (width 0.15) (layer F.Cu) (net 21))
 (segment (start 190.75 104.1) (end 191.65 104.1) (width 0.15) (layer F.Cu) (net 22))
 (segment (start 169.85 105) (end 170.75 105) (width 0.15) (layer F.Cu) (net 23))
 (segment (start 169.85 104.1) (end 170.75 104.1) (width 0.15) (layer F.Cu) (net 24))
 (segment (start 150.1 106) (end 149.9 105.6) (width 0.15) (layer F.Cu) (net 25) (status 30))
 (segment (start 194 105.8) (end 194.2 105.3) (width 0.15) (layer B.Cu) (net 25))
 (segment (start 150.2 105.8) (end 194 105.8) (width 0.15) (layer B.Cu) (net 25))
 (segment (start 150 105.6) (end 150.2 105.8) (width 0.15) (layer B.Cu) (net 25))
 (segment (start 149.4 104.9) (end 150 105.6) (width 0.15) (layer B.Cu) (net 25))
 (via (at 149.4 104.9) (size 0.5) (drill 0.3) (layers F.Cu B.Cu) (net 25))
 (segment (start 149.9 105.6) (end 149.4 104.9) (width 0.15) (layer F.Cu) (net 25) (status 10))
 (segment (start 193.15 105) (end 194 105) (width 0.15) (layer F.Cu) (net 25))
 (via (at 194.2 105.3) (size 0.5) (drill 0.3) (layers F.Cu B.Cu) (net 25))
 (segment (start 194 105) (end 194.2 105.3) (width 0.15) (layer F.Cu) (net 25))
 (segment (start 150.7 105.3) (end 193 105.3) (width 0.15) (layer B.Cu) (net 26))
 (segment (start 151.1 105.8) (end 150.7 105.3) (width 0.15) (layer F.Cu) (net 26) (status 10))
 (via (at 150.7 105.3) (size 0.5) (drill 0.3) (layers F.Cu B.Cu) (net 26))
 (via (at 194.2 104.1) (size 0.5) (drill 0.3) (layers F.Cu B.Cu) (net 26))
 (segment (start 194.2 104.1) (end 193.35 104.1) (width 0.15) (layer F.Cu) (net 26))
 (segment (start 193 105.3) (end 194.2 104.1) (width 0.15) (layer B.Cu) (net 26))
 (segment (start 151.5 105.8) (end 151.1 105.8) (width 0.15) (layer F.Cu) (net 26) (status 30))
 (segment (start 172.45 105) (end 173.35 105) (width 0.15) (layer F.Cu) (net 27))
 (segment (start 172.45 104.1) (end 173.35 104.1) (width 0.15) (layer F.Cu) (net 28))
 (segment (start 175.05 105) (end 175.95 105) (width 0.15) (layer F.Cu) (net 29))
 (segment (start 175.05 104.1) (end 175.95 104.1) (width 0.15) (layer F.Cu) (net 30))
 (segment (start 177.65 105) (end 178.65 105) (width 0.15) (layer F.Cu) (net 31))
 (segment (start 177.65 104.1) (end 178.65 104.1) (width 0.15) (layer F.Cu) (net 32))
 (segment (start 180.35 105) (end 181.25 105) (width 0.15) (layer F.Cu) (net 33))
 (segment (start 180.35 104.1) (end 181.25 104.1) (width 0.15) (layer F.Cu) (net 34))
 (segment (start 182.95 105) (end 183.85 105) (width 0.15) (layer F.Cu) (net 35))
 (segment (start 182.95 104.1) (end 183.85 104.1) (width 0.15) (layer F.Cu) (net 36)))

